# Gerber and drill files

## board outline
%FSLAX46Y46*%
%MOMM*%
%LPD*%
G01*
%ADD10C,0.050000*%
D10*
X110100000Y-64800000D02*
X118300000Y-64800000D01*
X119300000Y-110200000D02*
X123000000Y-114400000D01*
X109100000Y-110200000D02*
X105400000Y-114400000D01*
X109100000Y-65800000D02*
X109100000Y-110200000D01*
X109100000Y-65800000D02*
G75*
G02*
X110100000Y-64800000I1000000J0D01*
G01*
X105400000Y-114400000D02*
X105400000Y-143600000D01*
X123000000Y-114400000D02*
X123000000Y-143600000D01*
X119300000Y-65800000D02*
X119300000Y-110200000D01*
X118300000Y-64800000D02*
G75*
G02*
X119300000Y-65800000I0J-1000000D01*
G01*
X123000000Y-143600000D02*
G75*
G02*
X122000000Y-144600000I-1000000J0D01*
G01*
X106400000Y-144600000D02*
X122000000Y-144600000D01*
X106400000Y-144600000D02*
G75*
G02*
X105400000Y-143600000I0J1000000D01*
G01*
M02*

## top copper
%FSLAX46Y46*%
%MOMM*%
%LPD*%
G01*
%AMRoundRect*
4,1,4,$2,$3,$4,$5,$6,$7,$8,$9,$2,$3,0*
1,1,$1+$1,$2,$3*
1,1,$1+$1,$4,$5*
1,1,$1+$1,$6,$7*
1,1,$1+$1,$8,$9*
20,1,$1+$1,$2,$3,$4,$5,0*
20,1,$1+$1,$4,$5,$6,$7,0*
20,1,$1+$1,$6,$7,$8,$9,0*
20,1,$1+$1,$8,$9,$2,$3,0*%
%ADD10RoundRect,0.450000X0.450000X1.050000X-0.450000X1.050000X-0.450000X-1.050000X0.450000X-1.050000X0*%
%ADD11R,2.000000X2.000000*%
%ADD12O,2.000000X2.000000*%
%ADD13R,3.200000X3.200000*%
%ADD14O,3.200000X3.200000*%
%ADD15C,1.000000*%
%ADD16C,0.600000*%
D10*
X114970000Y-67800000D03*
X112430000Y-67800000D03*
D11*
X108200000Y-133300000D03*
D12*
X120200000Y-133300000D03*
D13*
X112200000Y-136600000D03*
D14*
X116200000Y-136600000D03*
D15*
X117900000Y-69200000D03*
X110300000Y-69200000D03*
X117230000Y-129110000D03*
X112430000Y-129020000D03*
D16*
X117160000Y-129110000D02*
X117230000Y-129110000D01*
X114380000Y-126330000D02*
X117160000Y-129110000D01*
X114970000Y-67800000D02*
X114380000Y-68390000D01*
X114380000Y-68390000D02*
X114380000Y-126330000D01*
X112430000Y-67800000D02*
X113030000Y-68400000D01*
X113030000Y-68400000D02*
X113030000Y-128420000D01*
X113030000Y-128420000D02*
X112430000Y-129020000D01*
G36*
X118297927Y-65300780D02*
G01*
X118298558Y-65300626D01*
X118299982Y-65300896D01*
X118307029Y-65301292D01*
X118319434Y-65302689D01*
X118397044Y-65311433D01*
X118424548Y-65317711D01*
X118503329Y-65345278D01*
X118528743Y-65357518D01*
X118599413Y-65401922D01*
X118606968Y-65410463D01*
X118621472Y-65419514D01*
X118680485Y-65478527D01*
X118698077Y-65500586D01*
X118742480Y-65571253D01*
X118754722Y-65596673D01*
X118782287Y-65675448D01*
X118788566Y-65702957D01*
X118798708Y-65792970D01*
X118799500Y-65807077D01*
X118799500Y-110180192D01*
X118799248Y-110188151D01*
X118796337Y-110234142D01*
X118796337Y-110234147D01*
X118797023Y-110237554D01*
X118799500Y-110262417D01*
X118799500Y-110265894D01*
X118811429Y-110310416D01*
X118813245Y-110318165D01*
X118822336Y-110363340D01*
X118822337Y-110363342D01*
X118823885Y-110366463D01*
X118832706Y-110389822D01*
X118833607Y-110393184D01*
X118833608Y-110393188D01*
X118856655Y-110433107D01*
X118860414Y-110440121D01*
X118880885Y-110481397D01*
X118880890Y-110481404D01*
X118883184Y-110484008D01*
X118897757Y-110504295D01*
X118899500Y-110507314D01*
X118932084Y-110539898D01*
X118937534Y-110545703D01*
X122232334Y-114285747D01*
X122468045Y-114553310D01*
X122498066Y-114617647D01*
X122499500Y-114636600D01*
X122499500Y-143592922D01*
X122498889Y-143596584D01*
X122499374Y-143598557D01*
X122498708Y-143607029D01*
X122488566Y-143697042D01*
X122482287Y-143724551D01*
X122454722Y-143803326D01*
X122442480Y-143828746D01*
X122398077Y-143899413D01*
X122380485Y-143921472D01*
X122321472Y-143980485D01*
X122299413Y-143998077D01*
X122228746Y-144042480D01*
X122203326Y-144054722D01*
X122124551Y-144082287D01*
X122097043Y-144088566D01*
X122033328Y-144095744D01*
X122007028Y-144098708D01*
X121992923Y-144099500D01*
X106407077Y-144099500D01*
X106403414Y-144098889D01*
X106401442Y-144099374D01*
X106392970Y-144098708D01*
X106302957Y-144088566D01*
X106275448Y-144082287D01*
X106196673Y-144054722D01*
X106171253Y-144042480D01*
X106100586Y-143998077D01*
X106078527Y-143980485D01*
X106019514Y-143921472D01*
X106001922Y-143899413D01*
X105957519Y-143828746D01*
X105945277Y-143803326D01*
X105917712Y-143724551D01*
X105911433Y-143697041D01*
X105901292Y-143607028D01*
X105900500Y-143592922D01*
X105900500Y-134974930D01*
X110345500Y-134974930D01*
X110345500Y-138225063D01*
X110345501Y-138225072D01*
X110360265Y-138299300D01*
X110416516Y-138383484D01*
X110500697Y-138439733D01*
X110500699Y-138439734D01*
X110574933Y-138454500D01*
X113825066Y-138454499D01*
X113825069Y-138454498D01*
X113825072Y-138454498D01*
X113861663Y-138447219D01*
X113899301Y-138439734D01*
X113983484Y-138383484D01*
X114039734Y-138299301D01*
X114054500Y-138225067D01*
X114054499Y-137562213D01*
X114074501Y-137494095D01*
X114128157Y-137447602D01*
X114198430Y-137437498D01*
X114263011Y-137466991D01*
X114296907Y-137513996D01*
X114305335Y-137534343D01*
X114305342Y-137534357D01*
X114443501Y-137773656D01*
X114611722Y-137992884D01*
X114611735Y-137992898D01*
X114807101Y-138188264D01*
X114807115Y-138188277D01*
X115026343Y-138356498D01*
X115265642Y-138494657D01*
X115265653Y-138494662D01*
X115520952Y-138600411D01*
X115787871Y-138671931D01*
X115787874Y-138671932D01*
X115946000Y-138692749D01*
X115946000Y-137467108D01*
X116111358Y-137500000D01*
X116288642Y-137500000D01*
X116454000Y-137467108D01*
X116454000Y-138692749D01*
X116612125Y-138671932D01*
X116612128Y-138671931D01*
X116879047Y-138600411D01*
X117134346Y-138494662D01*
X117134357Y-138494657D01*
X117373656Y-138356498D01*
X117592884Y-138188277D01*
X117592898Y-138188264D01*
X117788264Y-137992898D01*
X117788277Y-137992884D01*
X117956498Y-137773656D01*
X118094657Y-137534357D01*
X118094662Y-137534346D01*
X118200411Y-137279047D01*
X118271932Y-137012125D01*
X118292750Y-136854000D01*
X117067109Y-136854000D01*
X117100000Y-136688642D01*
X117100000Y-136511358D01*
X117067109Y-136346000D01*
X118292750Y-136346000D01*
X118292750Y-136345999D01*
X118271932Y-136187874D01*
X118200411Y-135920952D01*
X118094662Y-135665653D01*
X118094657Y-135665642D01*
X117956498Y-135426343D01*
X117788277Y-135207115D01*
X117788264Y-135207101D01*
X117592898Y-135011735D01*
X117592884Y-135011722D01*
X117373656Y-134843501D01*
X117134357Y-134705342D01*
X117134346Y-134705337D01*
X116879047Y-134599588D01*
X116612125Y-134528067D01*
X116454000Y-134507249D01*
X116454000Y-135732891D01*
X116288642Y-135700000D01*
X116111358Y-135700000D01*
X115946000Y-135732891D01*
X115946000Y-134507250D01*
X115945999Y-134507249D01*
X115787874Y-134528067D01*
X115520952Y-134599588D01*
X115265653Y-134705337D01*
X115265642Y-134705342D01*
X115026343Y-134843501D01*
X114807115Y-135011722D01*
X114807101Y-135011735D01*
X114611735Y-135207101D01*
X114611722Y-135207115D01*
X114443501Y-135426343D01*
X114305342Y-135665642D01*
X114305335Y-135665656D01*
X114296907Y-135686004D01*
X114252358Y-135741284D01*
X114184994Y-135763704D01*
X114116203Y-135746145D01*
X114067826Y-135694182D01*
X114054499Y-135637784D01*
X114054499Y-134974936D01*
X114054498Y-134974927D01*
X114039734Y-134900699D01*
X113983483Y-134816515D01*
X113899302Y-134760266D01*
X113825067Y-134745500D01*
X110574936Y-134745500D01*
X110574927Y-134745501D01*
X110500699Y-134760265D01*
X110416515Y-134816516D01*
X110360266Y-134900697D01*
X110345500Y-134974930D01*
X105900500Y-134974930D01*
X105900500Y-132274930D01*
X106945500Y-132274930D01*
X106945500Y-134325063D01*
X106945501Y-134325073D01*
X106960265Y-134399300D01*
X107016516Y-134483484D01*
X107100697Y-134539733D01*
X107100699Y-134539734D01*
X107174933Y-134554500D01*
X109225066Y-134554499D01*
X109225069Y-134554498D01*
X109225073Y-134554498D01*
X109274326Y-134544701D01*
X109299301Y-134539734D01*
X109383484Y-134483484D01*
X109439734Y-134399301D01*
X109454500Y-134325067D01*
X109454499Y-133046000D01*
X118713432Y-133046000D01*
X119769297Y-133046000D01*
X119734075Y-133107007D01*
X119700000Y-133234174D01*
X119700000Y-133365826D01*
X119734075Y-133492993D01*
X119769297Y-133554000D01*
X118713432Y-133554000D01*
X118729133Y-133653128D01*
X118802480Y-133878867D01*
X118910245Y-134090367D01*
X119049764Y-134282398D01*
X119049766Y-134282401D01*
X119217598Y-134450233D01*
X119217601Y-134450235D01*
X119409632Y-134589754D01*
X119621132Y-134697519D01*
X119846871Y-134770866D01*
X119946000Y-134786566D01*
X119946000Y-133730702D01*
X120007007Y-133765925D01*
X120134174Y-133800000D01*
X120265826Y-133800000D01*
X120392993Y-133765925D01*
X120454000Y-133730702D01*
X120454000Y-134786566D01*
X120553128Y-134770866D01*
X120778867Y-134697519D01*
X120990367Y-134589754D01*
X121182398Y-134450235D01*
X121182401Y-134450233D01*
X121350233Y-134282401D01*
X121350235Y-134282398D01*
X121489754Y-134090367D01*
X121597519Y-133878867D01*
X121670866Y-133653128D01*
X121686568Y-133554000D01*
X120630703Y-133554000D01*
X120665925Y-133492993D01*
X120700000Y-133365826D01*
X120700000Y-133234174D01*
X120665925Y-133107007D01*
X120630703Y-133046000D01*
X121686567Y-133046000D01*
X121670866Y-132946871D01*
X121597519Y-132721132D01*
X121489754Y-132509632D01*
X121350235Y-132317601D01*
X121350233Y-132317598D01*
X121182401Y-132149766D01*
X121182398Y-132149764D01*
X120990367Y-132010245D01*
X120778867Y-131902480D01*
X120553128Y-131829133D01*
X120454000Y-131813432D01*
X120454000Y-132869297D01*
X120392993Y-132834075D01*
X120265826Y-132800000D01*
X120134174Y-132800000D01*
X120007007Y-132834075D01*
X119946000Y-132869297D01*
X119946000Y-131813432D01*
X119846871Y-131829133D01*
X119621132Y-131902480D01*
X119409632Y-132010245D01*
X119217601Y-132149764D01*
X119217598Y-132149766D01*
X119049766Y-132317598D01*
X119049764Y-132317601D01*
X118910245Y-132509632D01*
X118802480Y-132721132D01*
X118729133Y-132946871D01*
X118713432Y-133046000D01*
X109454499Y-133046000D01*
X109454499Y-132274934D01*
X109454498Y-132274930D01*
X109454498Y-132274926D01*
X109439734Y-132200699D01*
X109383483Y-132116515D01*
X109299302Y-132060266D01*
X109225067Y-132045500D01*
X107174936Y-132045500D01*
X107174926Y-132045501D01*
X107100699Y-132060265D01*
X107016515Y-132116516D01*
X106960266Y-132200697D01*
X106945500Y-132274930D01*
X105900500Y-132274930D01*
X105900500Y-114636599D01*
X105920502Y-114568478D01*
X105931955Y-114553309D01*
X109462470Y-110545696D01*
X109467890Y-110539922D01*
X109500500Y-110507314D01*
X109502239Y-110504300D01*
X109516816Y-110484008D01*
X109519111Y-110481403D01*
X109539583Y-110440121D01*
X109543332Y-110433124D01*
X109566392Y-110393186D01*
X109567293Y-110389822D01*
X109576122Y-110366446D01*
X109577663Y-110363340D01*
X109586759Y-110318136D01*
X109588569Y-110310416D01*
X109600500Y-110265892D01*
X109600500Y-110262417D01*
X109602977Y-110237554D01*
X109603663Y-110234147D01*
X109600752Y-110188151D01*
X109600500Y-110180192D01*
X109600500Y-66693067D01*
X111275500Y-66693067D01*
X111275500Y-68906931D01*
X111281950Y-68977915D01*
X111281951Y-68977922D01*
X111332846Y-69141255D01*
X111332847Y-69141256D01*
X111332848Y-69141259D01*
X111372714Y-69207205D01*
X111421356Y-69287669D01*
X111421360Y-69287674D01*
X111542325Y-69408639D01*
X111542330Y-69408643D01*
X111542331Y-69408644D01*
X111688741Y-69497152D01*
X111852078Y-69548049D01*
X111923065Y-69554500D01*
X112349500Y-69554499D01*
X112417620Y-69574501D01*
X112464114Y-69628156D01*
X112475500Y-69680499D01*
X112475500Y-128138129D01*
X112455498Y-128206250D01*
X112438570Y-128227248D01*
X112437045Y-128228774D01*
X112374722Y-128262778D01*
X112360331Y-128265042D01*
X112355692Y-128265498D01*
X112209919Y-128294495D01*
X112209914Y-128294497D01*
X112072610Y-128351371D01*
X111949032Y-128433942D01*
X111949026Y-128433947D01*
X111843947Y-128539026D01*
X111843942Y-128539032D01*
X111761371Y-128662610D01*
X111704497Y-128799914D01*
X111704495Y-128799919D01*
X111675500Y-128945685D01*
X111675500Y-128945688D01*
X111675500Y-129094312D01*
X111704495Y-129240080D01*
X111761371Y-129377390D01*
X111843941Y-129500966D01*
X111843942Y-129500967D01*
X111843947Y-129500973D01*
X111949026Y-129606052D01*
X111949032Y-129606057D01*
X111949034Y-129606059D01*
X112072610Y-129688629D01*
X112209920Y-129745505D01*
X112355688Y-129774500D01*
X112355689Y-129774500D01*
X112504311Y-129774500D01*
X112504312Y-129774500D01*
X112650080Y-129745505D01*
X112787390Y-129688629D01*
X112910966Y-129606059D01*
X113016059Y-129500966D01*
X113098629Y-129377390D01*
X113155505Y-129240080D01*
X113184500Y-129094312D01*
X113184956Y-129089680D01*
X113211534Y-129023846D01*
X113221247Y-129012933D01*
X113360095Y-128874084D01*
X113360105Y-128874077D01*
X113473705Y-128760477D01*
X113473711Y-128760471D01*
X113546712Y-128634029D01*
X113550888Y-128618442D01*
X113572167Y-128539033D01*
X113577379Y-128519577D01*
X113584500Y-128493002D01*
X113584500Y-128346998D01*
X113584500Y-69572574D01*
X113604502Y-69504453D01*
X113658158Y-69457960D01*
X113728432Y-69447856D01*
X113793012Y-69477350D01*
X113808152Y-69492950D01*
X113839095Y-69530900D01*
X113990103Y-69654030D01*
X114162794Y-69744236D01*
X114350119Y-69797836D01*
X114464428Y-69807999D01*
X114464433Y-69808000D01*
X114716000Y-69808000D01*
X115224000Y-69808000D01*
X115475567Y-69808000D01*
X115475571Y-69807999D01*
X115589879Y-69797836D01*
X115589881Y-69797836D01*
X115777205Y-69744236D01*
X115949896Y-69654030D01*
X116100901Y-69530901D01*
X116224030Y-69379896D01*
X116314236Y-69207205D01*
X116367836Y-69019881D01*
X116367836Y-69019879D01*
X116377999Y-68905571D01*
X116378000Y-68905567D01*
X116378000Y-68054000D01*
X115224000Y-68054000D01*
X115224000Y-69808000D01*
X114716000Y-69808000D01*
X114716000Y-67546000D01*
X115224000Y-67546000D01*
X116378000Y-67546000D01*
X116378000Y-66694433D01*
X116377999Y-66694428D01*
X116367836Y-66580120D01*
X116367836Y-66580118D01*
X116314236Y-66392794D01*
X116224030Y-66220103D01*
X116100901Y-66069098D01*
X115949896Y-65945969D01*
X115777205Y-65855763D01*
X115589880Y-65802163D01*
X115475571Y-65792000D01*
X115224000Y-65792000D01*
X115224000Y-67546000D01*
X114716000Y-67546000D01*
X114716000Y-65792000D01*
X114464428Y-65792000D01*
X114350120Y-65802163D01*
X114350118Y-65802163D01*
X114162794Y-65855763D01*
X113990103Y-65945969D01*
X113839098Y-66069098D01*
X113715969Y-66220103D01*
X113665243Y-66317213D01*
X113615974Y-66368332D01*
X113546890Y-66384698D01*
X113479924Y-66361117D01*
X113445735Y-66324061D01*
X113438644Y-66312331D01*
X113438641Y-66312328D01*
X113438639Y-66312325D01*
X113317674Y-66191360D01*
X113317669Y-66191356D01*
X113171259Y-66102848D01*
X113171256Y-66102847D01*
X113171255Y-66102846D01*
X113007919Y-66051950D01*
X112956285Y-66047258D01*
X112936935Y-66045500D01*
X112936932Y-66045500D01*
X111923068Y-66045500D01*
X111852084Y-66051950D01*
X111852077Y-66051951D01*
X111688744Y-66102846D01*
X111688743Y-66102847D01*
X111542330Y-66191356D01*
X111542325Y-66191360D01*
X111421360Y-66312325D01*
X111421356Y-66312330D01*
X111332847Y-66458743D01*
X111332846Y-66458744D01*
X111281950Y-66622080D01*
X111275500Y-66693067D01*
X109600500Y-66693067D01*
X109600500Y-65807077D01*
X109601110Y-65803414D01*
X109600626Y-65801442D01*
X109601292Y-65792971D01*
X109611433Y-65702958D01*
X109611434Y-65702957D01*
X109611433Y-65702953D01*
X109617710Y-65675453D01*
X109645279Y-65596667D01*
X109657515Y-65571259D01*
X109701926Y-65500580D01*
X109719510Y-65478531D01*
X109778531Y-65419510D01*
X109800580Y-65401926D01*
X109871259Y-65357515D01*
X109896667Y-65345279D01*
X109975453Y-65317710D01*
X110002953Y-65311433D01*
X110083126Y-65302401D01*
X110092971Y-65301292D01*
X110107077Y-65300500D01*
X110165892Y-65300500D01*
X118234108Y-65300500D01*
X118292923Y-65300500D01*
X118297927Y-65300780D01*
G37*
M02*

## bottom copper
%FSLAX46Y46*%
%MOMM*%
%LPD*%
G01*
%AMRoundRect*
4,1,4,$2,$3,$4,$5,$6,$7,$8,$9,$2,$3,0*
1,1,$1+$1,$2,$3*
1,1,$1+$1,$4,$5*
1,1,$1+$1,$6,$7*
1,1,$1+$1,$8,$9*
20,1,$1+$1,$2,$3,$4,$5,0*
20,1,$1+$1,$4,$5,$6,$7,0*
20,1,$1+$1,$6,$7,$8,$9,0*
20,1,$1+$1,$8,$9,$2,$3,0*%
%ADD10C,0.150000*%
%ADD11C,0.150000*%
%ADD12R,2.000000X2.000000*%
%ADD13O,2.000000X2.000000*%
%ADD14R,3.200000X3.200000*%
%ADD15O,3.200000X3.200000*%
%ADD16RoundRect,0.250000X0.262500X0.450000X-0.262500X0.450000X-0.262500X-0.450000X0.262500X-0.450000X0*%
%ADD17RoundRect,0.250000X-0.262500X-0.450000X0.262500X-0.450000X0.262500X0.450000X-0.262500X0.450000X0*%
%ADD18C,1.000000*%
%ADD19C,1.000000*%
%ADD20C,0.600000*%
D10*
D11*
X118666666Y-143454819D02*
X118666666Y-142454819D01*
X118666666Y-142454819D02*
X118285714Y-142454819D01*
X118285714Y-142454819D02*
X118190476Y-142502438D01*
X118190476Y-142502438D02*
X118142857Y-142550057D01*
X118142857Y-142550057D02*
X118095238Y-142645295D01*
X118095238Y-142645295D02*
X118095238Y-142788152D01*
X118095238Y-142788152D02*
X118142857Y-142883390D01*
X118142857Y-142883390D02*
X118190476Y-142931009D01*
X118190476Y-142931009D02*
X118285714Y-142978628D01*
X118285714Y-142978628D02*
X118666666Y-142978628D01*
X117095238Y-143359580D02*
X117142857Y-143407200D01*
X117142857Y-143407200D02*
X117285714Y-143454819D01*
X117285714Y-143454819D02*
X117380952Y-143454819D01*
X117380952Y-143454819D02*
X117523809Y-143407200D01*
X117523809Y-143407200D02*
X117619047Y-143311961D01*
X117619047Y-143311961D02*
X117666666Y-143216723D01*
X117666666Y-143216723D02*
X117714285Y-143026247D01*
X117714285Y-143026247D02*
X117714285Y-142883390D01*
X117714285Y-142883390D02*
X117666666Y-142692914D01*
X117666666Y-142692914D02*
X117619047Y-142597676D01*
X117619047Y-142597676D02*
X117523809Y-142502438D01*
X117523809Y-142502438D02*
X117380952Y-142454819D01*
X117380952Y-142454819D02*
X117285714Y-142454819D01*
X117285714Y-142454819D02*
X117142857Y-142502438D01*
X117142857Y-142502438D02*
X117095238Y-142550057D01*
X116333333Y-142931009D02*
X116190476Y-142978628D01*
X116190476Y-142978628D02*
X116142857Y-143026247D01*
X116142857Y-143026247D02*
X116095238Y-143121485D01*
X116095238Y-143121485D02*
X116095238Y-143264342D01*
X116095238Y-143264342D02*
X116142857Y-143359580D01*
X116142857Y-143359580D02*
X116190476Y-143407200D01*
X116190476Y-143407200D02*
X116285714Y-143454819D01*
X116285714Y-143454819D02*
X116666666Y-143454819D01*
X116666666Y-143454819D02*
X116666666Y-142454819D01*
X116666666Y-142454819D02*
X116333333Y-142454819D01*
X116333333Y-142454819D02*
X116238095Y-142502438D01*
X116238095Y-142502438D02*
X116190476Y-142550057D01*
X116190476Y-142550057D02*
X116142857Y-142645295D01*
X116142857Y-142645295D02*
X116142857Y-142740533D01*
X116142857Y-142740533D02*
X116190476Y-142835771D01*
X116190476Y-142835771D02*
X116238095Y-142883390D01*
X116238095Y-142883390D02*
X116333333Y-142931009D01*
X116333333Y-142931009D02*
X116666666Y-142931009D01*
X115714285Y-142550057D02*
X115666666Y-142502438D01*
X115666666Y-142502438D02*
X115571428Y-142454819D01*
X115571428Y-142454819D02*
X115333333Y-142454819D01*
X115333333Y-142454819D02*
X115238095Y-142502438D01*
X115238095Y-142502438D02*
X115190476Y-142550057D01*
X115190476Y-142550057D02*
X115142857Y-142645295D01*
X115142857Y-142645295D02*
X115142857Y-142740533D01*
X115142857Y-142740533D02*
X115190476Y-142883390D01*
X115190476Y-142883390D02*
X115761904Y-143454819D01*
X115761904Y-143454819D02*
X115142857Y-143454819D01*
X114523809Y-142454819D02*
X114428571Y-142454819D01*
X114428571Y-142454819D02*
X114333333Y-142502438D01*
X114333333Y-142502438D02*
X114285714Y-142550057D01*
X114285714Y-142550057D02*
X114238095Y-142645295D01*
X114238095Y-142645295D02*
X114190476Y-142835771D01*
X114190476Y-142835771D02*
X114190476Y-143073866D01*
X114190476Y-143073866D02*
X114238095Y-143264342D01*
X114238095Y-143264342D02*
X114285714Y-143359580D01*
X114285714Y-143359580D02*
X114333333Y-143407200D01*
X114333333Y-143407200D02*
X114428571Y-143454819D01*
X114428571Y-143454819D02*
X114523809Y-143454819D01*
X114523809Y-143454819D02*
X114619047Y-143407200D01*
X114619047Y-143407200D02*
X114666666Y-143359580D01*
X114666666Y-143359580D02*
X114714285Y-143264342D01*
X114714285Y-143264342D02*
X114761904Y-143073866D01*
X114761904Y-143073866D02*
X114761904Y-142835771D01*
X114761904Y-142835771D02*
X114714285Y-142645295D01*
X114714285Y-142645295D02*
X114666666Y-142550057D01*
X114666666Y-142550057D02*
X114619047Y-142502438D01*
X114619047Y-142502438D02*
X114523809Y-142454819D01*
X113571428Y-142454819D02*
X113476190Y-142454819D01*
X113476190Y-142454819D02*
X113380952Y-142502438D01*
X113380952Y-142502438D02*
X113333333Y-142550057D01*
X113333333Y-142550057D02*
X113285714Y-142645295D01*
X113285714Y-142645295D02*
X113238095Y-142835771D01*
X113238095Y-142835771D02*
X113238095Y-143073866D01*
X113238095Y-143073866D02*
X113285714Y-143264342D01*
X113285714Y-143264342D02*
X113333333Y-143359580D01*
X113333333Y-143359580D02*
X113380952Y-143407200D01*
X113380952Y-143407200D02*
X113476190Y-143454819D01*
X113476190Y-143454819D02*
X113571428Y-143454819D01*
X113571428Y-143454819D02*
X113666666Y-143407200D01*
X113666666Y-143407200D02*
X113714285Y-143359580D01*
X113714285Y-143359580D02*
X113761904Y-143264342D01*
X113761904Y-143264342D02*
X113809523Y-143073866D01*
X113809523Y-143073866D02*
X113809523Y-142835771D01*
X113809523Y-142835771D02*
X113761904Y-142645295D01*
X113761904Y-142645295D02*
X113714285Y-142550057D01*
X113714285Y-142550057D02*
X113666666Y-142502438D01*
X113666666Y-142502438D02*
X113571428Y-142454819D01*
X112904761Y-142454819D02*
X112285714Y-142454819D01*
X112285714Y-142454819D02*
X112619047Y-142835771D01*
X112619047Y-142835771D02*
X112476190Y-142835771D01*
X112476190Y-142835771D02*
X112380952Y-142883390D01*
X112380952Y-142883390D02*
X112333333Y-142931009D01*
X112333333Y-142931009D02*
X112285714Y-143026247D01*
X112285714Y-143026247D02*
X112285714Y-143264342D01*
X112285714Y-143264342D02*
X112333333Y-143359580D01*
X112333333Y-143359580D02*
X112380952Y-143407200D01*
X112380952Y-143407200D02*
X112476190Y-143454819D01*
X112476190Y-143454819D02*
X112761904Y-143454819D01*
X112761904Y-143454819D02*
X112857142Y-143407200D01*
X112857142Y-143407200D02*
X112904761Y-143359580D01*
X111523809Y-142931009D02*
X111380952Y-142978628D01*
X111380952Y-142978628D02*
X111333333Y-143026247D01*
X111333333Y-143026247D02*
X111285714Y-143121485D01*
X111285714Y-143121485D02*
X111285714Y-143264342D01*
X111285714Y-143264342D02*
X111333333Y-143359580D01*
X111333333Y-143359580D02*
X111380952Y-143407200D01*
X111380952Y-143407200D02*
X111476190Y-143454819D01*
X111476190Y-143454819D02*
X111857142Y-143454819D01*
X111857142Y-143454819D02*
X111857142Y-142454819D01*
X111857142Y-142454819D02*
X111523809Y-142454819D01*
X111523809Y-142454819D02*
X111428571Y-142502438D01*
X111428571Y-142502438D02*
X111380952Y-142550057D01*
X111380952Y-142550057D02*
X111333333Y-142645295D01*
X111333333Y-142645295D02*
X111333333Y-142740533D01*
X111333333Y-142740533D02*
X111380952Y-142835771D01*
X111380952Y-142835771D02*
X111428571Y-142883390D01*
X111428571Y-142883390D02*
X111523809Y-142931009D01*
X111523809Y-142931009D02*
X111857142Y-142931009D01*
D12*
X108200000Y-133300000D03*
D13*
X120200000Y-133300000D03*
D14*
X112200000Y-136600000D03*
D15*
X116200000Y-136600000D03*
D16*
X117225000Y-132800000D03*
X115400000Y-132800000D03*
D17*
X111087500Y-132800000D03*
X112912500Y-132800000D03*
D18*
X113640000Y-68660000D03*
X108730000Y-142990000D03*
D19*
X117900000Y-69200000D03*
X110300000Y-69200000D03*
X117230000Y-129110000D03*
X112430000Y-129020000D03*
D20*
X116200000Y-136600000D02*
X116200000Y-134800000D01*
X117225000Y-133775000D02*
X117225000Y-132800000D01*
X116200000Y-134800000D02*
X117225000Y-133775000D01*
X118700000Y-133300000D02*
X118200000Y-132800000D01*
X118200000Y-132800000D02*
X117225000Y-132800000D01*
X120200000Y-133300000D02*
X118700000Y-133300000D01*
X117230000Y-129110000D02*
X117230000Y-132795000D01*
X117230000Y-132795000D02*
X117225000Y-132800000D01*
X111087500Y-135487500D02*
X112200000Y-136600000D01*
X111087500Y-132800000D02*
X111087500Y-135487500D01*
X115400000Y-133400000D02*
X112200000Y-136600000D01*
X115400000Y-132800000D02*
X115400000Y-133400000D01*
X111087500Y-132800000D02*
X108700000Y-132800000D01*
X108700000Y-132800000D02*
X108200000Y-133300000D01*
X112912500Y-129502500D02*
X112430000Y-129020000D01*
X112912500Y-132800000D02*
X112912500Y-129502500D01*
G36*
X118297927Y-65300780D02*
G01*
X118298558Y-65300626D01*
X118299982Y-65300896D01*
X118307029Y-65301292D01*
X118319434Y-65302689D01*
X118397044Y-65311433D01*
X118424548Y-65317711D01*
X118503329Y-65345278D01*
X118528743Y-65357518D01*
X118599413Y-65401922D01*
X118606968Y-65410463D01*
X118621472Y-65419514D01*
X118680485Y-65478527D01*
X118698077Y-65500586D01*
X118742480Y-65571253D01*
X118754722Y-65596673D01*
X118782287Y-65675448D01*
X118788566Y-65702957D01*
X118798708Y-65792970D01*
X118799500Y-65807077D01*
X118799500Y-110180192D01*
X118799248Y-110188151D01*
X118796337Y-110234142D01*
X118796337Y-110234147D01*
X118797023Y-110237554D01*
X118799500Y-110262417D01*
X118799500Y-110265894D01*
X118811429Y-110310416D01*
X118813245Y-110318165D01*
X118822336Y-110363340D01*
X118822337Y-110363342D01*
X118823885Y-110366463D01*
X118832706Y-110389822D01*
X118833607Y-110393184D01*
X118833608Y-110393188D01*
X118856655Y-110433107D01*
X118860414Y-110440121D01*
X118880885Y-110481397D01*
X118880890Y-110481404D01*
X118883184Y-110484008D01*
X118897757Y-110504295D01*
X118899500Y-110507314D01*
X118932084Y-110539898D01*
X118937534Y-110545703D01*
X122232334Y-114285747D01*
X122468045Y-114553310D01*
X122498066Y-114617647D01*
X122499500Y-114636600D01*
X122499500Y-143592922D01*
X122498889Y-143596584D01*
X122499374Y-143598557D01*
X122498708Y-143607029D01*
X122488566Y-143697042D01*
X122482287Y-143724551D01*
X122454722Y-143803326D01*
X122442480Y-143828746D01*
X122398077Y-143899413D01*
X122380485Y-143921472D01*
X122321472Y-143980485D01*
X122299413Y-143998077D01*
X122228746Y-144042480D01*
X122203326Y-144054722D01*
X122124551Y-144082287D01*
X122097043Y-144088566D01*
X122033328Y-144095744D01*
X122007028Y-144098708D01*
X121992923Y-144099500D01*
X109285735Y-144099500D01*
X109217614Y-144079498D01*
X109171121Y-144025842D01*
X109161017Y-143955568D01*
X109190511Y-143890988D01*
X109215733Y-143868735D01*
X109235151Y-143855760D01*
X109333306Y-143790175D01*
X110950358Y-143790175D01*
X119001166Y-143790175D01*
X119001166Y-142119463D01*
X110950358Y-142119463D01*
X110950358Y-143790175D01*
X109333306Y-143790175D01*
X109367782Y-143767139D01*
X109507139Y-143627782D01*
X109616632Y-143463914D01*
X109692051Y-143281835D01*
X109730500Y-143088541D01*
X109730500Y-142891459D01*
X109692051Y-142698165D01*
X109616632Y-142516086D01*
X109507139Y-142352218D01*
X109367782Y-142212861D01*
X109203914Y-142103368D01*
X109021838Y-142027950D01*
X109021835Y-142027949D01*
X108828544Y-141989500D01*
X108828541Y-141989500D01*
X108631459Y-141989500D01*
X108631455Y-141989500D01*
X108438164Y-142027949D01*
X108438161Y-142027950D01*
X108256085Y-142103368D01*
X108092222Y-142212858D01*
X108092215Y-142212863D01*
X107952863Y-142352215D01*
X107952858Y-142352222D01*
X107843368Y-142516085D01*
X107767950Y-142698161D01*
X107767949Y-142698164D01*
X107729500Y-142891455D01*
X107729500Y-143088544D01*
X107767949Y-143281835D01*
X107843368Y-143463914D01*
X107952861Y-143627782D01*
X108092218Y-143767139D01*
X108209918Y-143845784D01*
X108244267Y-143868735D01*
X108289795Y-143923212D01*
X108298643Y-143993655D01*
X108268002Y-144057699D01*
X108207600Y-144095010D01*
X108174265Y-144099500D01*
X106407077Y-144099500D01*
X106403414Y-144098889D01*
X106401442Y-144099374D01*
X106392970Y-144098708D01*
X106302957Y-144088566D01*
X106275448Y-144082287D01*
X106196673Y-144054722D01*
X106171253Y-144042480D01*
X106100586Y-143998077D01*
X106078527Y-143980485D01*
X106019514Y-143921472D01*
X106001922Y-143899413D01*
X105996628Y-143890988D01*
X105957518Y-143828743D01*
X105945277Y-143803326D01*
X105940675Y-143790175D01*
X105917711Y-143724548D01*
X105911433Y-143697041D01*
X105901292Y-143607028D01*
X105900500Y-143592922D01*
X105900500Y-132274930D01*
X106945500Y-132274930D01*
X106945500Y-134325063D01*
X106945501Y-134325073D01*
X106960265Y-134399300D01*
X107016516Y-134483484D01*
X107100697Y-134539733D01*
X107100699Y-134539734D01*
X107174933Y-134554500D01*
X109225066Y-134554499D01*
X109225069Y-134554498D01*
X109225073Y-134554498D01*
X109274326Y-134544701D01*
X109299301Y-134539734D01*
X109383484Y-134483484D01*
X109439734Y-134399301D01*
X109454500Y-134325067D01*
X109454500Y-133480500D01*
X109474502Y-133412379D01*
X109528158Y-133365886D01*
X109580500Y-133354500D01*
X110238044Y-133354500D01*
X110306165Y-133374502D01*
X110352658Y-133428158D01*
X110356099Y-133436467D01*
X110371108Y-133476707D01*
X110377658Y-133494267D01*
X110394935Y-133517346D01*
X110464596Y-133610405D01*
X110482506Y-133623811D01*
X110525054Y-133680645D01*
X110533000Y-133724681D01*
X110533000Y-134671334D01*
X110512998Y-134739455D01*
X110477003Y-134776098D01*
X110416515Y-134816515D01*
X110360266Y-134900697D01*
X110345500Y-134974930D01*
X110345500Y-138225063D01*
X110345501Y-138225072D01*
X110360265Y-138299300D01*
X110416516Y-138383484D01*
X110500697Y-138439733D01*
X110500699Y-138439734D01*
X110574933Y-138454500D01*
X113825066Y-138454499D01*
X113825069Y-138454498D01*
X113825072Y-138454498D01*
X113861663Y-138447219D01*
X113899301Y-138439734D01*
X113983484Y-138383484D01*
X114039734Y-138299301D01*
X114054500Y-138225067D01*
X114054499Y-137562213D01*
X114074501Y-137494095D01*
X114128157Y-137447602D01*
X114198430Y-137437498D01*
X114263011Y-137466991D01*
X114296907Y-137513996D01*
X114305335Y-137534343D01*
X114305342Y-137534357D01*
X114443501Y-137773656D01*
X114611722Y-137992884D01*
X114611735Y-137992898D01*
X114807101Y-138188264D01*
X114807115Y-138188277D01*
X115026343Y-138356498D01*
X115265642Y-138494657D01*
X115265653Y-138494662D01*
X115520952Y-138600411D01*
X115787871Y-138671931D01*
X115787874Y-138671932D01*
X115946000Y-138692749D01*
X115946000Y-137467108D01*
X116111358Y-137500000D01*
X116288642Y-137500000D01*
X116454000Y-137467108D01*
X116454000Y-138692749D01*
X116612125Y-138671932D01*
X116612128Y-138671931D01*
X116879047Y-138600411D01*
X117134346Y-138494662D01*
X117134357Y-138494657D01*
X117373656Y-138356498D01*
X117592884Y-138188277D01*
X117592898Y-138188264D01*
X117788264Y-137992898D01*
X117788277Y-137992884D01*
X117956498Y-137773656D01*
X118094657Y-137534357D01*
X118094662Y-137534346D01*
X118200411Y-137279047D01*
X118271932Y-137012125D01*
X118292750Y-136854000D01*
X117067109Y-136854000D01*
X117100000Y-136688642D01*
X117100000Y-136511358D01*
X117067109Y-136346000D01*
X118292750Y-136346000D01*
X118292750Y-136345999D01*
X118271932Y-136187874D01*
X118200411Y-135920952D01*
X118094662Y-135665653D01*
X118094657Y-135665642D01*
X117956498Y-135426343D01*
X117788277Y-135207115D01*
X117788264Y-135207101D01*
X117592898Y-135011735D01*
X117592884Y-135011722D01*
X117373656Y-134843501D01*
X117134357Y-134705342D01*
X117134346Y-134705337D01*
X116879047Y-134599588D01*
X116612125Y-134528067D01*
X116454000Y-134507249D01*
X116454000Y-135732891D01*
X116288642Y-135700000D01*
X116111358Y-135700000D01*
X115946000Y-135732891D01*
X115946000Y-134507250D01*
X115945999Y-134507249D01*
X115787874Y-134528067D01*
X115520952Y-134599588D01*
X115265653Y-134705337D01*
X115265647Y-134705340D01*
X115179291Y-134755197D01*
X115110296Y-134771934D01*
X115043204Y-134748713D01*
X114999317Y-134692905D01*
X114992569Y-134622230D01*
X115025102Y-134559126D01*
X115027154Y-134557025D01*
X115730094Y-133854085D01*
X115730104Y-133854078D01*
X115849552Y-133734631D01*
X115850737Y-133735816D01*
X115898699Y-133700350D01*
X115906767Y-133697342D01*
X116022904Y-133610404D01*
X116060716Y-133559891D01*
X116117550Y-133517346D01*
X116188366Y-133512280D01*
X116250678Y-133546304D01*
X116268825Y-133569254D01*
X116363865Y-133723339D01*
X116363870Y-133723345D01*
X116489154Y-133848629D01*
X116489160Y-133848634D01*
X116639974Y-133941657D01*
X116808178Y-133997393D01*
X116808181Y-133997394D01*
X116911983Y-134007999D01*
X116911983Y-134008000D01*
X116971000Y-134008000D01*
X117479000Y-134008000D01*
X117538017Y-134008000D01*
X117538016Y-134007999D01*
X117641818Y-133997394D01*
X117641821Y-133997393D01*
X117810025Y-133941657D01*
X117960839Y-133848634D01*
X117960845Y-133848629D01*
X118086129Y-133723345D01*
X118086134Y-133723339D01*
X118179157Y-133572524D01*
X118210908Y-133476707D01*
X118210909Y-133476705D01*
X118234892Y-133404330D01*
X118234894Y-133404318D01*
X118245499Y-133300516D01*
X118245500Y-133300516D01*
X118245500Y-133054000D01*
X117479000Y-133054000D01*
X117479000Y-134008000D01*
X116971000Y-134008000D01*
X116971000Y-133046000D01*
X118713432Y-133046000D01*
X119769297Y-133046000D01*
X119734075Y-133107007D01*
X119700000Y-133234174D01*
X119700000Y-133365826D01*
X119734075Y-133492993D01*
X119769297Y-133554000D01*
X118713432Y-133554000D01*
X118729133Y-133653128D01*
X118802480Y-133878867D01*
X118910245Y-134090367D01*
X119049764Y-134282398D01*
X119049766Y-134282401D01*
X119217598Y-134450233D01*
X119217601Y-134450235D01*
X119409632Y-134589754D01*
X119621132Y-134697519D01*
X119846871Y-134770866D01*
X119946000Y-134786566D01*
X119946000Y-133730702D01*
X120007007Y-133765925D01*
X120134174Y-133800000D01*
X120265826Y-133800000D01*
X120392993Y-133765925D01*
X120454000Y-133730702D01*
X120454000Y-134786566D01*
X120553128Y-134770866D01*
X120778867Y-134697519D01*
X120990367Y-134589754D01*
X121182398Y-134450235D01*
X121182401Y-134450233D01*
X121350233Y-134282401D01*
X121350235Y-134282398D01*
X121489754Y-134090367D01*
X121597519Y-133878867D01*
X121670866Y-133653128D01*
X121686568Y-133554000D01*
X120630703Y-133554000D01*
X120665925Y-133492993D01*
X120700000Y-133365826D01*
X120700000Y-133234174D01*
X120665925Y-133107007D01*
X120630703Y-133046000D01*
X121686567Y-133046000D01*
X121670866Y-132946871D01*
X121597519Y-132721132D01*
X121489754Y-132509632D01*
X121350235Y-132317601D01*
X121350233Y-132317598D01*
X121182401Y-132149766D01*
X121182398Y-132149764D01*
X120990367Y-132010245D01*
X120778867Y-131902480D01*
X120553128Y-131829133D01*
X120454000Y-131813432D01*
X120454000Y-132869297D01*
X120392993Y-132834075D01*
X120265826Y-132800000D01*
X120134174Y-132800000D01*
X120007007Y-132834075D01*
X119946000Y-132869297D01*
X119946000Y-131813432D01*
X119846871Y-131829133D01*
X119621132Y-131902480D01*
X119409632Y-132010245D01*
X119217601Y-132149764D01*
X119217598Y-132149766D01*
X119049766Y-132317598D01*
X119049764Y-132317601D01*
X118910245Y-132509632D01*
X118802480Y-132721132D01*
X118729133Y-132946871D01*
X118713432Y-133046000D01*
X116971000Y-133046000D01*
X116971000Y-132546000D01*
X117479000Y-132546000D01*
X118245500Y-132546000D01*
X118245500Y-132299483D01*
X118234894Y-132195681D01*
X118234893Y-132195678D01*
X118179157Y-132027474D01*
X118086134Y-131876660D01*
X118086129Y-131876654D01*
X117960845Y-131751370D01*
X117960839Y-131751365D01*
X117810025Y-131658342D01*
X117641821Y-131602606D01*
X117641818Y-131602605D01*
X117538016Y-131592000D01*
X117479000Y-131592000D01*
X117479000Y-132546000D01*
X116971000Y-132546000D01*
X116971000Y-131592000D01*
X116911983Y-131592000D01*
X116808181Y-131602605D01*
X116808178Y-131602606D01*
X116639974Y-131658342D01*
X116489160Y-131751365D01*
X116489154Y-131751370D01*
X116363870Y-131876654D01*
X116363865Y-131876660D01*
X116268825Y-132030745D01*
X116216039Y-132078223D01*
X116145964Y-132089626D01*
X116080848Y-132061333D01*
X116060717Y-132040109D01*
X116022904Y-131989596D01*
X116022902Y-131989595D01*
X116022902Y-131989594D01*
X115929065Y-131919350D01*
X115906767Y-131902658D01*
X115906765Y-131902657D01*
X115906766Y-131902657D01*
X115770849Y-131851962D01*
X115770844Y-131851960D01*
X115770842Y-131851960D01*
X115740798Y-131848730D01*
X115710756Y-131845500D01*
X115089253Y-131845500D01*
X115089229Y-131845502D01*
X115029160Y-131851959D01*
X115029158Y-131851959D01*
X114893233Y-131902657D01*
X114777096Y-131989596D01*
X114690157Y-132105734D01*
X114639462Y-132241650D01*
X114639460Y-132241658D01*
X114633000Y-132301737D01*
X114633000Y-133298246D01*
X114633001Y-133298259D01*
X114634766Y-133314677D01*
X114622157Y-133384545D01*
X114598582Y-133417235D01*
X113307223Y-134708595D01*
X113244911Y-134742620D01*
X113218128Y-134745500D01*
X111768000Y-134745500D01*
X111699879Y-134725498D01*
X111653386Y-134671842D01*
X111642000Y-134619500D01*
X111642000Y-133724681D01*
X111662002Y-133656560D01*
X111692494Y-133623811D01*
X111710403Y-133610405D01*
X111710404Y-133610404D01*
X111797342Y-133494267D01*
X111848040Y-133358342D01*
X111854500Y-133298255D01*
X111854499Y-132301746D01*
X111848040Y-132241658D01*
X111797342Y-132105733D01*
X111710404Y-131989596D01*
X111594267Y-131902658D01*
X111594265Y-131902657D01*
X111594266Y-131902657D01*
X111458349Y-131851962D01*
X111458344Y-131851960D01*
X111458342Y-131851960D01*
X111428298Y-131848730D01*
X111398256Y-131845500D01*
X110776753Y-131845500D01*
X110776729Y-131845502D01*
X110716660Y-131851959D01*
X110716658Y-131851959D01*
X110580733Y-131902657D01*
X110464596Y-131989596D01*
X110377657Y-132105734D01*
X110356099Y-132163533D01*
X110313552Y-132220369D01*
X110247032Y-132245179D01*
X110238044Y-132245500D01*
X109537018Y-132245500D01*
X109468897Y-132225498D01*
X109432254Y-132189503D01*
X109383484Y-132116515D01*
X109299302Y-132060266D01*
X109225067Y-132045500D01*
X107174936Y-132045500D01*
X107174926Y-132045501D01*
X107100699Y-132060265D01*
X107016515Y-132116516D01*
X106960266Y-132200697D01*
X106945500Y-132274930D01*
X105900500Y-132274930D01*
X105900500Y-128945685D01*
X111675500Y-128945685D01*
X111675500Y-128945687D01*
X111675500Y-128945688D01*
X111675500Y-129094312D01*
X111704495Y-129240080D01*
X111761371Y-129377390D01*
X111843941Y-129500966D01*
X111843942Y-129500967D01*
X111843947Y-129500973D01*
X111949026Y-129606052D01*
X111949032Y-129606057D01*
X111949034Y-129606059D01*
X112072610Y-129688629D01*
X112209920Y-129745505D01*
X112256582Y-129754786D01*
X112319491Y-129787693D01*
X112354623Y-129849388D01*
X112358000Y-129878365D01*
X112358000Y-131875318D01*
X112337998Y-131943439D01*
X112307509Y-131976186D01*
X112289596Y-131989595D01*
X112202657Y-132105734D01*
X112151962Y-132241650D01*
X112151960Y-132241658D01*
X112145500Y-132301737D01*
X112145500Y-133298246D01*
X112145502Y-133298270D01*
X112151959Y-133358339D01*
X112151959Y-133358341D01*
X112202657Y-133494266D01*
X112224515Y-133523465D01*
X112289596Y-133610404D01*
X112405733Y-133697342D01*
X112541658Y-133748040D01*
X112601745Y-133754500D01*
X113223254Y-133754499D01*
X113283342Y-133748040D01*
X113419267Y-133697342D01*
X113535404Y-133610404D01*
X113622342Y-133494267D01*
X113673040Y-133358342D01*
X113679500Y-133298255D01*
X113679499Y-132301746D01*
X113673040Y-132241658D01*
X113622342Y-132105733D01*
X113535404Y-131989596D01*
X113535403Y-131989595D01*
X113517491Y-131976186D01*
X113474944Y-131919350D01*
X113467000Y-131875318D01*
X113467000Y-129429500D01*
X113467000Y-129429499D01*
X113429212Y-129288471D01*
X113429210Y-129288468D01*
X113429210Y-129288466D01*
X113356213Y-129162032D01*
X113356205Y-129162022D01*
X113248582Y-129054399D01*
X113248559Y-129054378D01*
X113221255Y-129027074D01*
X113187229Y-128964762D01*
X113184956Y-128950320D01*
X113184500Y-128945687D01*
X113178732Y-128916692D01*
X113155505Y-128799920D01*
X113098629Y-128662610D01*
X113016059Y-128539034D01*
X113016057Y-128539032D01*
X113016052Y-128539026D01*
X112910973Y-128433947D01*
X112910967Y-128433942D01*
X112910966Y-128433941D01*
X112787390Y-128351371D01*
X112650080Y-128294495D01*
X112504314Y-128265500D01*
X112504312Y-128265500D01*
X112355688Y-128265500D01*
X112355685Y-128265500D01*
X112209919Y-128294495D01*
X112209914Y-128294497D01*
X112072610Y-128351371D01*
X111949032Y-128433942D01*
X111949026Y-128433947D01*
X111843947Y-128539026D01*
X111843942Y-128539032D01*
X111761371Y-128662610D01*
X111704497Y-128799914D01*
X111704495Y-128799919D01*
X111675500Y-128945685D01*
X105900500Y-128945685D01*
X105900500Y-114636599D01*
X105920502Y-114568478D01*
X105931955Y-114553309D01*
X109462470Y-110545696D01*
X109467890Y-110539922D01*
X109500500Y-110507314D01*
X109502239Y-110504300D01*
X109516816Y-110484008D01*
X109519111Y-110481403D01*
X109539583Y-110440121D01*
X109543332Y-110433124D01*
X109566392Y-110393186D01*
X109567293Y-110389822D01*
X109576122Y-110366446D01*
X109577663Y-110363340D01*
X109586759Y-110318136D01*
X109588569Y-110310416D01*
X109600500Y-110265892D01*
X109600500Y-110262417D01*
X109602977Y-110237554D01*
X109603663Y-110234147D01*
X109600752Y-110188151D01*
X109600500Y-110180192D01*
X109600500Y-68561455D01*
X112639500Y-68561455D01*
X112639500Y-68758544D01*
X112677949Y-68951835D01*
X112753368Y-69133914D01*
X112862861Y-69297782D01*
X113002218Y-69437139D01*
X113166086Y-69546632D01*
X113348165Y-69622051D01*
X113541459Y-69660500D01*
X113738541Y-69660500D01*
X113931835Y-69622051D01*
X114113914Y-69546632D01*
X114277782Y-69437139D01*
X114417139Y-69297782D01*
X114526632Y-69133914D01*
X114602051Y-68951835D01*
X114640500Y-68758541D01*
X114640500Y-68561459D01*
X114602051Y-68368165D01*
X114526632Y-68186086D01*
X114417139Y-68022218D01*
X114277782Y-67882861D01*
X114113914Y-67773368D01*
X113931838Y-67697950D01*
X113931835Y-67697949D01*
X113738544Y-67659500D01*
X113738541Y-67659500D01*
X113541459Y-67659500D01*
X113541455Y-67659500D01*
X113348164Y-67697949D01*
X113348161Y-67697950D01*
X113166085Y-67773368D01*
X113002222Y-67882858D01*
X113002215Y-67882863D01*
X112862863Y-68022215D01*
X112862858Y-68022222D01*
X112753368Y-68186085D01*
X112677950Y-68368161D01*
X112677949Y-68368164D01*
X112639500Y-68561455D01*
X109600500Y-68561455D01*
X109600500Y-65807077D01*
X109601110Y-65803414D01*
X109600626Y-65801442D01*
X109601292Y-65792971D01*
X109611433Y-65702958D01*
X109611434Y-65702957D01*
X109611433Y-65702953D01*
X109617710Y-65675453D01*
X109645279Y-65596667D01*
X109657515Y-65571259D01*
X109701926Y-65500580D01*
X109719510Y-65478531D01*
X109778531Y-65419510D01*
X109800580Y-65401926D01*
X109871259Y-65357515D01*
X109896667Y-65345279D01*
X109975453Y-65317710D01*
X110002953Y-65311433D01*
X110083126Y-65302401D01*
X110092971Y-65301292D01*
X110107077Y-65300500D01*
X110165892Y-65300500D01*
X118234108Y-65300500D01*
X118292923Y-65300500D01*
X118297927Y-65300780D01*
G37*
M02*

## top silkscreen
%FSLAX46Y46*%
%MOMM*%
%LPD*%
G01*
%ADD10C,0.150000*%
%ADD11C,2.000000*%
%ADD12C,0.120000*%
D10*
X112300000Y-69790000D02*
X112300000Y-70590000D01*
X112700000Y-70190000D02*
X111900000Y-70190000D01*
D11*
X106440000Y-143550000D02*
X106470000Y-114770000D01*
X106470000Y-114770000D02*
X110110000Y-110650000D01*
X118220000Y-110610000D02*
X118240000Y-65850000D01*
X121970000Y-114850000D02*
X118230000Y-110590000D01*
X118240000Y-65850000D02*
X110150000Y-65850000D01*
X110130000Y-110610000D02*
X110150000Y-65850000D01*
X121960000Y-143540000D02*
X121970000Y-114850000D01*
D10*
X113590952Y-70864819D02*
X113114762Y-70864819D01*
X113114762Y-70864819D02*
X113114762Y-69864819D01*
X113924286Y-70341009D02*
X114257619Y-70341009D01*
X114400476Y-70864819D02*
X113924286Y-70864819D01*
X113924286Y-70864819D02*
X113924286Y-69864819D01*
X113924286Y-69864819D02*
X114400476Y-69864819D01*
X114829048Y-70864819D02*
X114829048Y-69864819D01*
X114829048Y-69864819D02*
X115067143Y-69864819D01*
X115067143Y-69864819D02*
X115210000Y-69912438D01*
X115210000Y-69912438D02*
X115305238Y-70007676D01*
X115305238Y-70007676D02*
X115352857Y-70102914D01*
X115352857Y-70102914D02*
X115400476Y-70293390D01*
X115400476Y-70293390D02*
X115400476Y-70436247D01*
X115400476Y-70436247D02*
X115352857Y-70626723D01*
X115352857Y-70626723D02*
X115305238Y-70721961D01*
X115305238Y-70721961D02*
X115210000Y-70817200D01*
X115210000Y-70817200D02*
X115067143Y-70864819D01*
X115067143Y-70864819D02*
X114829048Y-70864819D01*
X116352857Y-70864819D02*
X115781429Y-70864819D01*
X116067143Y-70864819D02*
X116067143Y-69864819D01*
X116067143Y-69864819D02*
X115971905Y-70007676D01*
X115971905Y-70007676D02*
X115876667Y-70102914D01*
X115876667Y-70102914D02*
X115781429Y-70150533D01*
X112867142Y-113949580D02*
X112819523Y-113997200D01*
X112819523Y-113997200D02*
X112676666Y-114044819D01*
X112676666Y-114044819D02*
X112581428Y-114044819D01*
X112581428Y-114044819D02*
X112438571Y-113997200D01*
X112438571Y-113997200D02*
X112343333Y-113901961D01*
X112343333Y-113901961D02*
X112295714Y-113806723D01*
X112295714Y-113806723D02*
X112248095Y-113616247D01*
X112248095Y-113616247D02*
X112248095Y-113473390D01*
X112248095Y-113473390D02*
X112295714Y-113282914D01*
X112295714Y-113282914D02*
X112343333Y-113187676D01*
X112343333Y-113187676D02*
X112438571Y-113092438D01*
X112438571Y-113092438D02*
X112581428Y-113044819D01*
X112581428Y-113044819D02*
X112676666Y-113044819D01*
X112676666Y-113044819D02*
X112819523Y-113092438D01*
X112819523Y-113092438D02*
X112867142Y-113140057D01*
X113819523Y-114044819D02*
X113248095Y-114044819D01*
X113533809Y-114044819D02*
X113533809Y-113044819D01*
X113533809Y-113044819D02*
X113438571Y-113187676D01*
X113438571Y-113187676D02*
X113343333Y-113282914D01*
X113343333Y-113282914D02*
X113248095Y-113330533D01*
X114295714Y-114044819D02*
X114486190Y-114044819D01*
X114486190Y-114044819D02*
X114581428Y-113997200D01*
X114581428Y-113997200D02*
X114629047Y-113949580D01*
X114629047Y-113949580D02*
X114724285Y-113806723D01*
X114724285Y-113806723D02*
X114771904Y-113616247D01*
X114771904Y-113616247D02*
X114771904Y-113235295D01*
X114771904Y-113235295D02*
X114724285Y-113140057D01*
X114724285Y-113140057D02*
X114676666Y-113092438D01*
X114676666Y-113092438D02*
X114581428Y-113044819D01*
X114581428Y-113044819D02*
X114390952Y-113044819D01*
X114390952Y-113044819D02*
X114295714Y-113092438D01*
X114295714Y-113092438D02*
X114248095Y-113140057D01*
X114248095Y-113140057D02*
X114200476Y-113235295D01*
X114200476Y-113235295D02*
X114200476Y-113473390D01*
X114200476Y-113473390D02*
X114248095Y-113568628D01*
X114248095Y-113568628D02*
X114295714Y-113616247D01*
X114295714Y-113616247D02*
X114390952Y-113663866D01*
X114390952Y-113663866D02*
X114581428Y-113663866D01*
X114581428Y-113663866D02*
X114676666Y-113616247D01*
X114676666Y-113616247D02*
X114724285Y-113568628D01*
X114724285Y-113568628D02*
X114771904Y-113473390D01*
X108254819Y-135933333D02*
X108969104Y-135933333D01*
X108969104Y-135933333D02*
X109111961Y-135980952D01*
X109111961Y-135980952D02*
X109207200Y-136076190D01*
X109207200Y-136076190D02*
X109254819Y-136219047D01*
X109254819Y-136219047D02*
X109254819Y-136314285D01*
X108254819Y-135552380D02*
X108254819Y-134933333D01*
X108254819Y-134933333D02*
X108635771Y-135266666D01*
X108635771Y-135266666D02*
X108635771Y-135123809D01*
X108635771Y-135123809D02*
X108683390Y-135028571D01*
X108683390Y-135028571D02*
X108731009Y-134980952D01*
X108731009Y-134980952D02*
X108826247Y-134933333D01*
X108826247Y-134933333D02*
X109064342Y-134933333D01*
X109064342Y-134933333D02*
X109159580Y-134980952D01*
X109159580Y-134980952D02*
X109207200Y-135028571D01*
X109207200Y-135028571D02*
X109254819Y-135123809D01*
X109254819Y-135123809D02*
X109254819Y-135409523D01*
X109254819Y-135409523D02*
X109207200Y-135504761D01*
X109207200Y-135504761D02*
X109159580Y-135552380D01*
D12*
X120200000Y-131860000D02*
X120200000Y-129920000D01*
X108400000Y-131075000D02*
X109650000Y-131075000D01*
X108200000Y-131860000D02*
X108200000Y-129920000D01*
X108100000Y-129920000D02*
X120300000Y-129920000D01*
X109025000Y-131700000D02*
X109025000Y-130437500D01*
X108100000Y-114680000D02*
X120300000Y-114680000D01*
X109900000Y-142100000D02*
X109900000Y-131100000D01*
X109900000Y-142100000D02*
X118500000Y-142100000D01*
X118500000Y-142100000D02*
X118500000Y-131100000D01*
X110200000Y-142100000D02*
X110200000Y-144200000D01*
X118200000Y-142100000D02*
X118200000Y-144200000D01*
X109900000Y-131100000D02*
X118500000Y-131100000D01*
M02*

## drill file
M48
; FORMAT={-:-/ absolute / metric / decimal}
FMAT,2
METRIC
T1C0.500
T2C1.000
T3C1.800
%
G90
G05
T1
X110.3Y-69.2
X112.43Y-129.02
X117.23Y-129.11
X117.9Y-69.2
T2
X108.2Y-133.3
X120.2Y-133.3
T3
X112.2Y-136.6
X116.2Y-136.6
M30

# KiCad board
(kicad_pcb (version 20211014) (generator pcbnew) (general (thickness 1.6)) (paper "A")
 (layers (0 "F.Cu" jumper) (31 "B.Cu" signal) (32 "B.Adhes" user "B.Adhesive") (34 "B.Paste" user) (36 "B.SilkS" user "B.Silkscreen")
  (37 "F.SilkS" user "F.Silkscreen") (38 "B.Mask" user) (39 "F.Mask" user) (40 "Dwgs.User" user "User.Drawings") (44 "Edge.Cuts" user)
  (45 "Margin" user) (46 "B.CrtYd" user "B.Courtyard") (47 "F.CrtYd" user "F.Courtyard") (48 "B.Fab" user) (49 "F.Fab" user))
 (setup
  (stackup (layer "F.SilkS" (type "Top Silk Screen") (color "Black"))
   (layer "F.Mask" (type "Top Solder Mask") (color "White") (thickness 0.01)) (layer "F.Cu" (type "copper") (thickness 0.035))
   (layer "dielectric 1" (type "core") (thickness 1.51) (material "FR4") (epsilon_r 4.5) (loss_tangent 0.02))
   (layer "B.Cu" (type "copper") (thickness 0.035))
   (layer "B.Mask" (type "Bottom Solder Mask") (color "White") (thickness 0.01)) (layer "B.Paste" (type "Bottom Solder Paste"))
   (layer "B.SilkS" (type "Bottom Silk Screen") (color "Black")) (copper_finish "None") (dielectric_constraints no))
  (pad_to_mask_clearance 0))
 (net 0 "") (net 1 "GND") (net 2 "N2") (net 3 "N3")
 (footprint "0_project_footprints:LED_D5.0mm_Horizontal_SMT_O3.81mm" (layer "F.Cu") (at 113.7 67.8 180)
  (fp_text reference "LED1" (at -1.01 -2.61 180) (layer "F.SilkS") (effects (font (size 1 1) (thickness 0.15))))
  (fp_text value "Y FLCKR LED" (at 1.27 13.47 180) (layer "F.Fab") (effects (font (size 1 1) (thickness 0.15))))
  (pad "1" smd roundrect (at -1.27 0 180) (size 1.8 3) (layers "F.Cu" "F.Paste" "F.Mask") (roundrect_rratio 0.25) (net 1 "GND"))
  (pad "2" smd roundrect (at 1.27 0 180) (size 1.8 3) (layers "F.Cu" "F.Paste" "F.Mask") (roundrect_rratio 0.25) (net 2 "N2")))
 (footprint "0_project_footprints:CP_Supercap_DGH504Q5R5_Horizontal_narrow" (layer "F.Cu") (at 114.2 133.3 90)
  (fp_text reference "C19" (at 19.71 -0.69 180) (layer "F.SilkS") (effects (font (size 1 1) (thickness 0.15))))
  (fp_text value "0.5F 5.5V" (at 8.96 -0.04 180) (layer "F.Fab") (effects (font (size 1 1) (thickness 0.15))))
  (fp_line (start 1.44 6) (end 3.38 6) (layer "F.SilkS") (width 0.12))
  (fp_line (start 2.225 -5.8) (end 2.225 -4.55) (layer "F.SilkS") (width 0.12))
  (fp_line (start 1.44 -6) (end 3.38 -6) (layer "F.SilkS") (width 0.12))
  (fp_line (start 3.38 -6.1) (end 3.38 6.1) (layer "F.SilkS") (width 0.12))
  (fp_line (start 1.6 -5.175) (end 2.8625 -5.175) (layer "F.SilkS") (width 0.12))
  (fp_line (start 18.62 -6.1) (end 18.62 6.1) (layer "F.SilkS") (width 0.12))
  (pad "1" thru_hole rect (at 0 -6 90) (size 2 2) (drill 1) (layers *.Cu *.Mask) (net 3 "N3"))
  (pad "2" thru_hole oval (at 0 6 90) (size 2 2) (drill 1) (layers *.Cu *.Mask) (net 1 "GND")))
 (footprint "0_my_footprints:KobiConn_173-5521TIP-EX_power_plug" (layer "F.Cu") (at 114.2 136.6 90)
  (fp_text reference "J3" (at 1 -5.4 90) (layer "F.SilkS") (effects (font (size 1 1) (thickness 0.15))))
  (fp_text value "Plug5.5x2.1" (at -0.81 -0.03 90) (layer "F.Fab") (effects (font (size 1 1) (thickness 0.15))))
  (fp_line (start -5.5 -4.3) (end 5.5 -4.3) (layer "F.SilkS") (width 0.12))
  (fp_line (start -5.5 -4.3) (end -5.5 4.3) (layer "F.SilkS") (width 0.12))
  (fp_line (start -5.5 4.3) (end 5.5 4.3) (layer "F.SilkS") (width 0.12))
  (fp_line (start -5.5 -4) (end -7.6 -4) (layer "F.SilkS") (width 0.12))
  (fp_line (start -5.5 4) (end -7.6 4) (layer "F.SilkS") (width 0.12))
  (fp_line (start 5.5 -4.3) (end 5.5 4.3) (layer "F.SilkS") (width 0.12))
  (pad "1" thru_hole rect (at 0 -2 90) (size 3.2 3.2) (drill 1.8) (layers *.Cu *.Mask) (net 3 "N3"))
  (pad "2" thru_hole oval (at 0 2 90) (size 3.2 3.2) (drill 1.8) (layers *.Cu *.Mask) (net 1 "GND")))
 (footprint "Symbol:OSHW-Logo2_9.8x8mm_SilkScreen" (layer "B.Cu") (at 114.3 123.02 180)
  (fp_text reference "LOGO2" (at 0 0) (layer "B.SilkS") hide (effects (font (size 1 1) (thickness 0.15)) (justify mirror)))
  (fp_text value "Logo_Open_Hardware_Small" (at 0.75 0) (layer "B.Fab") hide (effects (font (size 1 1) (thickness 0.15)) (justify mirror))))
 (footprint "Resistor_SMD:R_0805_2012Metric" (layer "B.Cu") (at 116.3125 132.8 180)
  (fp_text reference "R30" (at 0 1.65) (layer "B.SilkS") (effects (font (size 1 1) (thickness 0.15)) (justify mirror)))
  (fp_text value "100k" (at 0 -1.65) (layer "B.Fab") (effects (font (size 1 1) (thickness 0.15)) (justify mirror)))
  (pad "1" smd roundrect locked (at -0.9125 0 180) (size 1.025 1.4) (layers "B.Cu" "B.Paste" "B.Mask") (roundrect_rratio 0.243902439)
   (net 1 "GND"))
  (pad "2" smd roundrect locked (at 0.9125 0 180) (size 1.025 1.4) (layers "B.Cu" "B.Paste" "B.Mask") (roundrect_rratio 0.243902439)
   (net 3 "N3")))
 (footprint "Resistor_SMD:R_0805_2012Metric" (layer "B.Cu") (at 112 132.8)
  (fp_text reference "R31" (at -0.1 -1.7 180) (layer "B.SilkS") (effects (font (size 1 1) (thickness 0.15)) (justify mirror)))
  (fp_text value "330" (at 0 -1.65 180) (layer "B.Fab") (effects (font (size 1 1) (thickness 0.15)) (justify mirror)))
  (pad "1" smd roundrect locked (at -0.9125 0) (size 1.025 1.4) (layers "B.Cu" "B.Paste" "B.Mask") (roundrect_rratio 0.243902439)
   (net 3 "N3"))
  (pad "2" smd roundrect locked (at 0.9125 0) (size 1.025 1.4) (layers "B.Cu" "B.Paste" "B.Mask") (roundrect_rratio 0.243902439)
   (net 2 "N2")))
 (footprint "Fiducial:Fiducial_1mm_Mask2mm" (layer "B.Cu") (at 113.64 68.66)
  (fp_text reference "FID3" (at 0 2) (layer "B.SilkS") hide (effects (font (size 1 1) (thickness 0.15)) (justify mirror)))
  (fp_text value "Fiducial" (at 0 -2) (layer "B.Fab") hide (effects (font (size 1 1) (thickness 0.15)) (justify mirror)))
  (pad "" smd circle locked (at 0 0) (size 1 1) (layers "B.Cu" "B.Mask") (solder_mask_margin 0.5) (clearance 0.5)))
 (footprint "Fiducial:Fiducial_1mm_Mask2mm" (layer "B.Cu") (at 108.73 142.99)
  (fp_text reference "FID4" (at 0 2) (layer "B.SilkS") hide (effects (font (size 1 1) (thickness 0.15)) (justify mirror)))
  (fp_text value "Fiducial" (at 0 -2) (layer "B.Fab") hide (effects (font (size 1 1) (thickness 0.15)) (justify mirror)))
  (pad "" smd circle locked (at 0 0) (size 1 1) (layers "B.Cu" "B.Mask") (solder_mask_margin 0.5) (clearance 0.5)))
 (gr_line (start 112.3 69.79) (end 112.3 70.59) (layer "F.SilkS") (width 0.15))
 (gr_line (start 112.7 70.19) (end 111.9 70.19) (layer "F.SilkS") (width 0.15))
 (gr_line (start 106.44 143.55) (end 106.47 114.77) (layer "F.SilkS") (width 2))
 (gr_line (start 106.47 114.77) (end 110.11 110.65) (layer "F.SilkS") (width 2))
 (gr_line (start 118.22 110.61) (end 118.24 65.85) (layer "F.SilkS") (width 2))
 (gr_line (start 121.97 114.85) (end 118.23 110.59) (layer "F.SilkS") (width 2))
 (gr_line (start 118.24 65.85) (end 110.15 65.85) (layer "F.SilkS") (width 2))
 (gr_line (start 110.13 110.61) (end 110.15 65.85) (layer "F.SilkS") (width 2))
 (gr_line (start 121.96 143.54) (end 121.97 114.85) (layer "F.SilkS") (width 2))
 (gr_line (start 110.1 64.8) (end 118.3 64.8) (layer "Edge.Cuts") (width 0.05))
 (gr_line (start 119.3 110.2) (end 123 114.4) (layer "Edge.Cuts") (width 0.05))
 (gr_line (start 109.1 110.2) (end 105.4 114.4) (layer "Edge.Cuts") (width 0.05))
 (gr_line (start 109.1 65.8) (end 109.1 110.2) (layer "Edge.Cuts") (width 0.05))
 (gr_arc (start 109.1 65.8) (mid 109.392893 65.092893) (end 110.1 64.8) (layer "Edge.Cuts") (width 0.05))
 (gr_line (start 105.4 114.4) (end 105.4 143.6) (layer "Edge.Cuts") (width 0.05))
 (gr_line (start 123 114.4) (end 123 143.6) (layer "Edge.Cuts") (width 0.05))
 (gr_line (start 119.3 65.8) (end 119.3 110.2) (layer "Edge.Cuts") (width 0.05))
 (gr_arc (start 118.3 64.8) (mid 119.007107 65.092893) (end 119.3 65.8) (layer "Edge.Cuts") (width 0.05))
 (gr_arc (start 123 143.6) (mid 122.707107 144.307107) (end 122 144.6) (layer "Edge.Cuts") (width 0.05))
 (gr_line (start 106.4 144.6) (end 122 144.6) (layer "Edge.Cuts") (width 0.05))
 (gr_arc (start 106.4 144.6) (mid 105.692893 144.307107) (end 105.4 143.6) (layer "Edge.Cuts") (width 0.05))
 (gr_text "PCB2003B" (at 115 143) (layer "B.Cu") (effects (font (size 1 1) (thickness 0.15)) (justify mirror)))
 (segment (start 117.16 129.11) (end 117.23 129.11) (width 0.6) (layer "F.Cu") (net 1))
 (segment (start 114.38 126.33) (end 117.16 129.11) (width 0.6) (layer "F.Cu") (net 1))
 (segment (start 114.97 67.8) (end 114.38 68.39) (width 0.6) (layer "F.Cu") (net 1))
 (segment (start 114.38 68.39) (end 114.38 126.33) (width 0.6) (layer "F.Cu") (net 1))
 (via (at 117.9 69.2) (size 1) (drill 0.5) (layers "F.Cu" "B.Cu") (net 1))
 (via (at 110.3 69.2) (size 1) (drill 0.5) (layers "F.Cu" "B.Cu") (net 1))
 (via (at 117.23 129.11) (size 1) (drill 0.5) (layers "F.Cu" "B.Cu") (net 1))
 (segment (start 116.2 136.6) (end 116.2 134.8) (width 0.6) (layer "B.Cu") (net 1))
 (segment (start 117.225 133.775) (end 117.225 132.8) (width 0.6) (layer "B.Cu") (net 1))
 (segment (start 116.2 134.8) (end 117.225 133.775) (width 0.6) (layer "B.Cu") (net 1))
 (segment (start 118.7 133.3) (end 118.2 132.8) (width 0.6) (layer "B.Cu") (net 1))
 (segment (start 118.2 132.8) (end 117.225 132.8) (width 0.6) (layer "B.Cu") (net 1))
 (segment (start 120.2 133.3) (end 118.7 133.3) (width 0.6) (layer "B.Cu") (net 1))
 (segment (start 117.23 129.11) (end 117.23 132.795) (width 0.6) (layer "B.Cu") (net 1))
 (segment (start 117.23 132.795) (end 117.225 132.8) (width 0.6) (layer "B.Cu") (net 1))
 (segment (start 111.0875 135.4875) (end 112.2 136.6) (width 0.6) (layer "B.Cu") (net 3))
 (segment (start 111.0875 132.8) (end 111.0875 135.4875) (width 0.6) (layer "B.Cu") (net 3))
 (segment (start 115.4 133.4) (end 112.2 136.6) (width 0.6) (layer "B.Cu") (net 3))
 (segment (start 115.4 132.8) (end 115.4 133.4) (width 0.6) (layer "B.Cu") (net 3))
 (segment (start 111.0875 132.8) (end 108.7 132.8) (width 0.6) (layer "B.Cu") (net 3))
 (segment (start 108.7 132.8) (end 108.2 133.3) (width 0.6) (layer "B.Cu") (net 3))
 (segment (start 112.43 67.8) (end 113.03 68.4) (width 0.6) (layer "F.Cu") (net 2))
 (segment (start 113.03 68.4) (end 113.03 128.42) (width 0.6) (layer "F.Cu") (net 2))
 (segment (start 113.03 128.42) (end 112.43 129.02) (width 0.6) (layer "F.Cu") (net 2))
 (via (at 112.43 129.02) (size 1) (drill 0.5) (layers "F.Cu" "B.Cu") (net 2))
 (segment (start 112.9125 129.5025) (end 112.43 129.02) (width 0.6) (layer "B.Cu") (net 2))
 (segment (start 112.9125 132.8) (end 112.9125 129.5025) (width 0.6) (layer "B.Cu") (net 2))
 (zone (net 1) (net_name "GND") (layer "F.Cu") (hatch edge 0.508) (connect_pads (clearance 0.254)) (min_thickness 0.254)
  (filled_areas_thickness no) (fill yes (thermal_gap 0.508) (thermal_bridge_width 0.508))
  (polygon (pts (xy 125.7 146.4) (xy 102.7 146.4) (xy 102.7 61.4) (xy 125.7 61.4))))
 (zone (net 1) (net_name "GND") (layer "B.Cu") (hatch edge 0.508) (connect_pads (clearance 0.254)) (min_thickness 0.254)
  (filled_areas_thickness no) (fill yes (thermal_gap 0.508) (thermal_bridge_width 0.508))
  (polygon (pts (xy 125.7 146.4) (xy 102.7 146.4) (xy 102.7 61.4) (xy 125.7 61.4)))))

